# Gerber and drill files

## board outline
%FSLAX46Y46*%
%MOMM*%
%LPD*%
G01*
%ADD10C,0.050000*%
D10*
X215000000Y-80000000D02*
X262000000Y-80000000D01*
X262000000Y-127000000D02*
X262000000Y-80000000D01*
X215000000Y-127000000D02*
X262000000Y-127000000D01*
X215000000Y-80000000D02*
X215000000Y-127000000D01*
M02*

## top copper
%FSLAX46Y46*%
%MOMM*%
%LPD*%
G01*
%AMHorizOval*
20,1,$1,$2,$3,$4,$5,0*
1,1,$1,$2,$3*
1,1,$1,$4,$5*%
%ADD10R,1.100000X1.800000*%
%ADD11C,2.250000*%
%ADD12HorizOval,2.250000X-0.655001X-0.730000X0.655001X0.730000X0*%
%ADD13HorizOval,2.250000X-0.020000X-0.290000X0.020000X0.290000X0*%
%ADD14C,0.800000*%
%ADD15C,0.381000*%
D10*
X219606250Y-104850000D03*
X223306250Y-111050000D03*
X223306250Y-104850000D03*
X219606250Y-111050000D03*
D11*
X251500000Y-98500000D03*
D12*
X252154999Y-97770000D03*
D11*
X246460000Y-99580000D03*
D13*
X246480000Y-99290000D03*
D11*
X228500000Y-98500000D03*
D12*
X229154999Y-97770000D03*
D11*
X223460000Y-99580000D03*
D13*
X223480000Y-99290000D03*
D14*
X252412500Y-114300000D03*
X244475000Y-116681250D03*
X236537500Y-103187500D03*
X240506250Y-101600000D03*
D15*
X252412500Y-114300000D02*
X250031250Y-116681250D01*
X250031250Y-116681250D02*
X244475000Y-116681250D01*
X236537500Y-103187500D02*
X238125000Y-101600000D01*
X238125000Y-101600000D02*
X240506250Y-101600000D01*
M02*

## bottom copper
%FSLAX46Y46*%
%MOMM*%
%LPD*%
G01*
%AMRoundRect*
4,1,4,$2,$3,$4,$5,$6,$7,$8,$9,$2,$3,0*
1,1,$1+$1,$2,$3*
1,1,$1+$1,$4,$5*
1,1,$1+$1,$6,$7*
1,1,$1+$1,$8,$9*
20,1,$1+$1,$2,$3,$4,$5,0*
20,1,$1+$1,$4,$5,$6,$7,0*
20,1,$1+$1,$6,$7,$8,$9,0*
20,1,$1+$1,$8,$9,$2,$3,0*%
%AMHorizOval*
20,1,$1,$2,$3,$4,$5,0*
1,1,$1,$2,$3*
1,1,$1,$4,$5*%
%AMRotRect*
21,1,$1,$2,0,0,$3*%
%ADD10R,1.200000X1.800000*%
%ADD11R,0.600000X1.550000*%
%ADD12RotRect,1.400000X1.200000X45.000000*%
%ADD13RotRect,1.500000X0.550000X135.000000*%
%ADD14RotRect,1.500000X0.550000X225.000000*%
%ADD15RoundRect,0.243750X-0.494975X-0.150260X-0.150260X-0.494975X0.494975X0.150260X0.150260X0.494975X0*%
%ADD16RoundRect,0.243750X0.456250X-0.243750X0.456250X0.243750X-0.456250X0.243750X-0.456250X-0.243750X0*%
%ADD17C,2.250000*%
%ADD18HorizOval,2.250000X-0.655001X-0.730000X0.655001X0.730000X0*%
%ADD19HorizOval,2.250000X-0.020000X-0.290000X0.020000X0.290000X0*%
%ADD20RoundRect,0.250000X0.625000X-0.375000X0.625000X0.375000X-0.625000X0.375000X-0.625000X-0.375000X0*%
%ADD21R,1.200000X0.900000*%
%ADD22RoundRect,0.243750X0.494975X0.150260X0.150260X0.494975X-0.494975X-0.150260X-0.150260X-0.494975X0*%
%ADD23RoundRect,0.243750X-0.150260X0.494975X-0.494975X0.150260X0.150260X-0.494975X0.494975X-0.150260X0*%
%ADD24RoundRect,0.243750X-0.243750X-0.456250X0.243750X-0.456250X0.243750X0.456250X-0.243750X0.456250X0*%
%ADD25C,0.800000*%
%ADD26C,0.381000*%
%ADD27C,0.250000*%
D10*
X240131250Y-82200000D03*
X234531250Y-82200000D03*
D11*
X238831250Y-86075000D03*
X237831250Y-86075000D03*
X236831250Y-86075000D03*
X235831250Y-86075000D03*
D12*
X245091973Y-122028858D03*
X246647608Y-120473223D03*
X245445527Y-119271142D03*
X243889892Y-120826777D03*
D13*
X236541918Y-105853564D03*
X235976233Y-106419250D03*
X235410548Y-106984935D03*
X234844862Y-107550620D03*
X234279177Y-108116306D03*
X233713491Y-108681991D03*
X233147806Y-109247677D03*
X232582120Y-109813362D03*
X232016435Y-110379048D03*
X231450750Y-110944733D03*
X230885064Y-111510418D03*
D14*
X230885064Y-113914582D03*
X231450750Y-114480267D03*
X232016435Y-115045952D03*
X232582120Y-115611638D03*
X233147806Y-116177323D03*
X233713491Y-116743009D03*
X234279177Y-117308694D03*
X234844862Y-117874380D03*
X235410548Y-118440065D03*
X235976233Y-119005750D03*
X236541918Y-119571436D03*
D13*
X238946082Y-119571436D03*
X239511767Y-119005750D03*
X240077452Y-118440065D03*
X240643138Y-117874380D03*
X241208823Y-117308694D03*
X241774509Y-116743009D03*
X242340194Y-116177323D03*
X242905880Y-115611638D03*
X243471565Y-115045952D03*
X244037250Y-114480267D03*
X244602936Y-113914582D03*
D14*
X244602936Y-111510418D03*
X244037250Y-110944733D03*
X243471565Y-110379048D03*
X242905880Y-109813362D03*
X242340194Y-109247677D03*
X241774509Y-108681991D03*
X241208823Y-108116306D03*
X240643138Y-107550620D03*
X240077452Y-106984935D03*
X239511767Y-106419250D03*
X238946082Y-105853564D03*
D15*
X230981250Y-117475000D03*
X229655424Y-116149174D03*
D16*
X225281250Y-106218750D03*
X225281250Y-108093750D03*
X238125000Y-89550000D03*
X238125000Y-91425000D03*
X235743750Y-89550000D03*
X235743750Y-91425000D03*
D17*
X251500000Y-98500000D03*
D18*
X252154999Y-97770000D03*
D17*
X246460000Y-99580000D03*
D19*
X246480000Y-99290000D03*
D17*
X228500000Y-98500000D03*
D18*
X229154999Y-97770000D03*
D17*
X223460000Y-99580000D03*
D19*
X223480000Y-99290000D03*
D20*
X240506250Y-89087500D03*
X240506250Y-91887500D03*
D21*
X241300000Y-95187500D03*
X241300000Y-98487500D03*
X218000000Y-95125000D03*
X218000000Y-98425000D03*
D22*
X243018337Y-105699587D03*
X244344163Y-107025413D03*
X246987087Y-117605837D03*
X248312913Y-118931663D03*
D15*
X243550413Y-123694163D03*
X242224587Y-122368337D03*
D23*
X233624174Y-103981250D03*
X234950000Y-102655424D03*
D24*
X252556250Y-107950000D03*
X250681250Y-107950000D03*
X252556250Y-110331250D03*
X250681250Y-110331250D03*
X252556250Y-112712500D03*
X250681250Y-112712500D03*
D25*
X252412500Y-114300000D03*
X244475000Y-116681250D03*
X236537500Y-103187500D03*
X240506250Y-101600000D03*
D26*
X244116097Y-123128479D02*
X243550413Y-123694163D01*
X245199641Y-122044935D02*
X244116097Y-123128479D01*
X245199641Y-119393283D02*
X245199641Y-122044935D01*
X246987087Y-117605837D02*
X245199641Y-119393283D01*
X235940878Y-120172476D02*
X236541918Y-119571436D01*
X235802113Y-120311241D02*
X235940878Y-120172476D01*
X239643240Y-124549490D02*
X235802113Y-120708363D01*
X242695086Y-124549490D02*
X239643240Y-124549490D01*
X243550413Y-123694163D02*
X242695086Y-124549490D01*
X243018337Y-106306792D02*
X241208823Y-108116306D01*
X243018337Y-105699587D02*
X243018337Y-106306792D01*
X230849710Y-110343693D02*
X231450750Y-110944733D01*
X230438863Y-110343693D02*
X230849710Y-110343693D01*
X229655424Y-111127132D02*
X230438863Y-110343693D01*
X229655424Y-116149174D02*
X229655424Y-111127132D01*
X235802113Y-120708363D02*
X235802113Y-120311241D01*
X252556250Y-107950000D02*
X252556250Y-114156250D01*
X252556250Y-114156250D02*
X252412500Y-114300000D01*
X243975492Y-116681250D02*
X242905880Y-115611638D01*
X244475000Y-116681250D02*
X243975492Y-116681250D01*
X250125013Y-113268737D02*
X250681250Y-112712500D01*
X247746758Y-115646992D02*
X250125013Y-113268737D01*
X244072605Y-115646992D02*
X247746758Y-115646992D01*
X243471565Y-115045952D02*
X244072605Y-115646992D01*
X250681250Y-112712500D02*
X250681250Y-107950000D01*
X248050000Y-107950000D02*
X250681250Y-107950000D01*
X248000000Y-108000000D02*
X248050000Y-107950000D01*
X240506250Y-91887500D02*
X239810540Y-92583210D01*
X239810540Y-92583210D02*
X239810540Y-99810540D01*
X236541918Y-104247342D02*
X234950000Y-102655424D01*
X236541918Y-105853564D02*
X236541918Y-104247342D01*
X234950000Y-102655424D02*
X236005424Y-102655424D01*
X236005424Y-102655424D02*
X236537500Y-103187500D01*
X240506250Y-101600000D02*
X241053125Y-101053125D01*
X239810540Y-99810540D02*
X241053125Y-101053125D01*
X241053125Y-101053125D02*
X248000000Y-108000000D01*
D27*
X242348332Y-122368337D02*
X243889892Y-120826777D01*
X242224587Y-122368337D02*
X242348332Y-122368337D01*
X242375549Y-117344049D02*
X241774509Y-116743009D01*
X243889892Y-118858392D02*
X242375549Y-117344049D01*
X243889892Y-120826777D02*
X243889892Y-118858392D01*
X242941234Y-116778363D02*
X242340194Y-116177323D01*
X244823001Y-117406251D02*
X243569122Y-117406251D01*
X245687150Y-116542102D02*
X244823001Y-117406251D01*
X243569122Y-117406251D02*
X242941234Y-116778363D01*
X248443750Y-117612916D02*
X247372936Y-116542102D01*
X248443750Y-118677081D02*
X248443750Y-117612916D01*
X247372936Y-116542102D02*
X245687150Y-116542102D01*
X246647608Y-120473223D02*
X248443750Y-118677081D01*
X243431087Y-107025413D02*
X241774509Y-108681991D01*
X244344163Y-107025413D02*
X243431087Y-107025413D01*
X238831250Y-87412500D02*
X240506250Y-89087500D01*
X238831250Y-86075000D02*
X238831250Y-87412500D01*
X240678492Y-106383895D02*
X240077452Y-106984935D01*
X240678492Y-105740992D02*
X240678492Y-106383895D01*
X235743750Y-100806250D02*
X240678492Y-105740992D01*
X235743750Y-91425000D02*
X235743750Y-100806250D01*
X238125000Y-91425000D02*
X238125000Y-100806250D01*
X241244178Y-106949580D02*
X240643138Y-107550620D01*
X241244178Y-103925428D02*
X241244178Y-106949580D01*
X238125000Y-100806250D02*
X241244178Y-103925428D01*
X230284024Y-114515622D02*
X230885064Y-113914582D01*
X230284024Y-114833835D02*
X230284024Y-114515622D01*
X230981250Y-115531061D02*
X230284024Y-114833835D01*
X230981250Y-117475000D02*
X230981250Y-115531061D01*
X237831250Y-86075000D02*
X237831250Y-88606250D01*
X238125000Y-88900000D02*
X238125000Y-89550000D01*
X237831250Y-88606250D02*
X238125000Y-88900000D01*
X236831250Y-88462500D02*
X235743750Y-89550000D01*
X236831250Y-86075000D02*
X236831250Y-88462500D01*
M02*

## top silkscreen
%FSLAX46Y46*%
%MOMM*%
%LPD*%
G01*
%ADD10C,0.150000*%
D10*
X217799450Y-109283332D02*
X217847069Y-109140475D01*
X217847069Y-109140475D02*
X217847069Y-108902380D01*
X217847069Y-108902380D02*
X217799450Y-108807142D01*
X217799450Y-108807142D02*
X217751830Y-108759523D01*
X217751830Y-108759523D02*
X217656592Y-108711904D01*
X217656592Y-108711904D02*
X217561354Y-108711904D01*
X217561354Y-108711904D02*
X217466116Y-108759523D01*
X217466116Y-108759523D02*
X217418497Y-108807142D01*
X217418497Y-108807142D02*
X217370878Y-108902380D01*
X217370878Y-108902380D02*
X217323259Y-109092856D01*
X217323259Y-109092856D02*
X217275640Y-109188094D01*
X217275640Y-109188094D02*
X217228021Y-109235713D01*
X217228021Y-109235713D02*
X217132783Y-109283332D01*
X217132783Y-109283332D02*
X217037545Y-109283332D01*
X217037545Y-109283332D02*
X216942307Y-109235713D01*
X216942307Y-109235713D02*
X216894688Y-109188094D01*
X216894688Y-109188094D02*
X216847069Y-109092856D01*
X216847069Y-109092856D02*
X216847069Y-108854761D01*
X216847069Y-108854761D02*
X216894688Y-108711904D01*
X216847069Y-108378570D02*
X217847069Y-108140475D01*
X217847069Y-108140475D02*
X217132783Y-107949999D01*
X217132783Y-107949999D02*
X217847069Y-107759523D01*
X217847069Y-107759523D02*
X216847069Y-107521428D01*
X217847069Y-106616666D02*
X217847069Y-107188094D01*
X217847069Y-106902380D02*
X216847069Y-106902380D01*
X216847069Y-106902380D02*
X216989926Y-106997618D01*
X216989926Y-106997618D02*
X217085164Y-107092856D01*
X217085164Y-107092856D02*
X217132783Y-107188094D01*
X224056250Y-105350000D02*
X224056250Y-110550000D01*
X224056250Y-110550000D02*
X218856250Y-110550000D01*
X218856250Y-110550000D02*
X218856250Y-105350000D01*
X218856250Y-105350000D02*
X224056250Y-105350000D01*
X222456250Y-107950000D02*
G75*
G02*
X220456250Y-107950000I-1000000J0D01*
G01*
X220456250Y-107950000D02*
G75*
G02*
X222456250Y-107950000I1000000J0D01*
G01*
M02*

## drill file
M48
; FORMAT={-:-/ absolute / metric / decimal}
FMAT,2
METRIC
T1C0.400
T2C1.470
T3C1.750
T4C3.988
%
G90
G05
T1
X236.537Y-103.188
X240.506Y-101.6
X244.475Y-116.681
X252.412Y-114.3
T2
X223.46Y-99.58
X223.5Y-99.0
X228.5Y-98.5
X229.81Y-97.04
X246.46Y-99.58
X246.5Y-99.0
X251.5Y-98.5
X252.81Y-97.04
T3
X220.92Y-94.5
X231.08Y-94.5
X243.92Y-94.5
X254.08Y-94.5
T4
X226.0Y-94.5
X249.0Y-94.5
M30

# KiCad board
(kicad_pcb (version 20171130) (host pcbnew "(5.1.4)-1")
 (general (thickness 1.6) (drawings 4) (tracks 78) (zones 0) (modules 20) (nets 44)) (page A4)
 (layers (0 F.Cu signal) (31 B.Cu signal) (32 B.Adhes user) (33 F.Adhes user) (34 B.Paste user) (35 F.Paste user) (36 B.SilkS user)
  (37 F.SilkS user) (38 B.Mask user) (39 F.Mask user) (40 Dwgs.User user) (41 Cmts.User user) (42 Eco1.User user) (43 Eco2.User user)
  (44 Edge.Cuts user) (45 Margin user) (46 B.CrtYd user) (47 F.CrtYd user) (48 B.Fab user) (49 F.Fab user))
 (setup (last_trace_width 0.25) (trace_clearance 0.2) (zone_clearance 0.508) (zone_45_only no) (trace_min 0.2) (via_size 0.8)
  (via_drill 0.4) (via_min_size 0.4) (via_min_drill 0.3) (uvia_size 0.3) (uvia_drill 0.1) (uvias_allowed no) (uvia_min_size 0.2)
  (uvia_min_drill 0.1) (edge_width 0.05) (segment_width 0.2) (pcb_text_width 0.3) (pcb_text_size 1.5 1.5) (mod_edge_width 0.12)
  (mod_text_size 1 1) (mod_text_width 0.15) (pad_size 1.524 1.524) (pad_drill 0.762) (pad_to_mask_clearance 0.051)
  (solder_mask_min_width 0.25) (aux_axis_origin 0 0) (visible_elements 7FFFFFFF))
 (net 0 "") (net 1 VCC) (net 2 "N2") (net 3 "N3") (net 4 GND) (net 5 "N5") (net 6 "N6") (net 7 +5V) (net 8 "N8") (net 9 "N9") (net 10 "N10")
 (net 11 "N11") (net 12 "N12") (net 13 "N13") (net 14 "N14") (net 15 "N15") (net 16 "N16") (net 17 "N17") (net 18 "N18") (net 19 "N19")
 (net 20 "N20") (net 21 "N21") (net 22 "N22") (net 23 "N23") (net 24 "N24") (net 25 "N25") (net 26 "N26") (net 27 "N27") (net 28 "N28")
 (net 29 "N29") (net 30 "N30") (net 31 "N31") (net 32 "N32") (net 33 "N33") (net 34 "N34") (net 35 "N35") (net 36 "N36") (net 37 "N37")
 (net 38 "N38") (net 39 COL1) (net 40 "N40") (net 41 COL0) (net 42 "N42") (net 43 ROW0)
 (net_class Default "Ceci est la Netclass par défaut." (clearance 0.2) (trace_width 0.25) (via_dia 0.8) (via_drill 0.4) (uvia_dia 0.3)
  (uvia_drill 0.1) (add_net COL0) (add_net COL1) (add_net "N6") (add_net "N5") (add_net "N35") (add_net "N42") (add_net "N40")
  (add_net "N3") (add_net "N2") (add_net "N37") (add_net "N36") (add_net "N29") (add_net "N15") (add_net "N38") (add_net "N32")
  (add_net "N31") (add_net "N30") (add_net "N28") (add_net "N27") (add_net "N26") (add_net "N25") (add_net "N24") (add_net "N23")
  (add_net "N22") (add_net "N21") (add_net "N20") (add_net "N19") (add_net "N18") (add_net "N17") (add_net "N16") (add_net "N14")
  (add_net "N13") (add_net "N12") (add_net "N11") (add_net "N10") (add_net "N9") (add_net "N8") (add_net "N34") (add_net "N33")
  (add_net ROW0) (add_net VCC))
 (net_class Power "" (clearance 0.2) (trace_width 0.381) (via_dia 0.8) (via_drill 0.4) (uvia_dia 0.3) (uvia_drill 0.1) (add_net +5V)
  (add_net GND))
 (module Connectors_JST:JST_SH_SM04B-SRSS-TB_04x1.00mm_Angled (layer B.Cu) (at 237.33125 84.1375)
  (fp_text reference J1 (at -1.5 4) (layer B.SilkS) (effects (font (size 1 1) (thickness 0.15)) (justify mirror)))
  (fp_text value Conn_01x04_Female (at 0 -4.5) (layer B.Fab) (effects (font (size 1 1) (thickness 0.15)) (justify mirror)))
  (pad "" smd rect (at 2.8 -1.9375) (size 1.2 1.8) (layers B.Cu B.Paste B.Mask))
  (pad "" smd rect (at -2.8 -1.9375) (size 1.2 1.8) (layers B.Cu B.Paste B.Mask))
  (pad 4 smd rect (at 1.5 1.9375) (size 0.6 1.55) (layers B.Cu B.Paste B.Mask) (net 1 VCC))
  (pad 3 smd rect (at 0.5 1.9375) (size 0.6 1.55) (layers B.Cu B.Paste B.Mask) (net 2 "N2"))
  (pad 2 smd rect (at -0.5 1.9375) (size 0.6 1.55) (layers B.Cu B.Paste B.Mask) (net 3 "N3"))
  (pad 1 smd rect (at -1.5 1.9375) (size 0.6 1.55) (layers B.Cu B.Paste B.Mask) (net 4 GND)))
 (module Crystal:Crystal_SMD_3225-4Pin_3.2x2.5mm (layer B.Cu) (at 245.26875 120.65 45)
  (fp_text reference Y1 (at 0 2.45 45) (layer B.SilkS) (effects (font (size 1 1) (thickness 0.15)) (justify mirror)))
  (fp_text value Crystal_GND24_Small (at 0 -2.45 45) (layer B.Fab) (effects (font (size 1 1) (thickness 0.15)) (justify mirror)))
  (pad 4 smd rect (at -1.1 0.85 45) (size 1.4 1.2) (layers B.Cu B.Paste B.Mask) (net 4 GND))
  (pad 3 smd rect (at 1.1 0.85 45) (size 1.4 1.2) (layers B.Cu B.Paste B.Mask) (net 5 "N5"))
  (pad 2 smd rect (at 1.1 -0.85 45) (size 1.4 1.2) (layers B.Cu B.Paste B.Mask) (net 4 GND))
  (pad 1 smd rect (at -1.1 -0.85 45) (size 1.4 1.2) (layers B.Cu B.Paste B.Mask) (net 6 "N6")))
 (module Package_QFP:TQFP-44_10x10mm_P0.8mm (layer B.Cu) (at 237.744 112.7125 225)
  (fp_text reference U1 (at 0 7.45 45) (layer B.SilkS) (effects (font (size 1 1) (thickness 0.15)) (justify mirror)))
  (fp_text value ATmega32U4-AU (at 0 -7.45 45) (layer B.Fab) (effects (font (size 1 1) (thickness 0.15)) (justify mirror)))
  (pad 44 smd rect (at -4 5.7 135) (size 1.5 0.55) (layers B.Cu B.Paste B.Mask) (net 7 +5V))
  (pad 43 smd rect (at -3.2 5.7 135) (size 1.5 0.55) (layers B.Cu B.Paste B.Mask) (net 4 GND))
  (pad 42 smd rect (at -2.4 5.7 135) (size 1.5 0.55) (layers B.Cu B.Paste B.Mask) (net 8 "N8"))
  (pad 41 smd rect (at -1.6 5.7 135) (size 1.5 0.55) (layers B.Cu B.Paste B.Mask) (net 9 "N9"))
  (pad 40 smd rect (at -0.8 5.7 135) (size 1.5 0.55) (layers B.Cu B.Paste B.Mask) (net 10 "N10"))
  (pad 39 smd rect (at 0 5.7 135) (size 1.5 0.55) (layers B.Cu B.Paste B.Mask) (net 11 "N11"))
  (pad 38 smd rect (at 0.8 5.7 135) (size 1.5 0.55) (layers B.Cu B.Paste B.Mask) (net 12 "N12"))
  (pad 37 smd rect (at 1.6 5.7 135) (size 1.5 0.55) (layers B.Cu B.Paste B.Mask) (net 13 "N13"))
  (pad 36 smd rect (at 2.4 5.7 135) (size 1.5 0.55) (layers B.Cu B.Paste B.Mask) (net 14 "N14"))
  (pad 35 smd rect (at 3.2 5.7 135) (size 1.5 0.55) (layers B.Cu B.Paste B.Mask) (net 4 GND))
  (pad 34 smd rect (at 4 5.7 135) (size 1.5 0.55) (layers B.Cu B.Paste B.Mask) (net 7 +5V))
  (pad 33 smd rect (at 5.7 4 225) (size 1.5 0.55) (layers B.Cu B.Paste B.Mask) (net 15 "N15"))
  (pad 32 smd rect (at 5.7 3.2 225) (size 1.5 0.55) (layers B.Cu B.Paste B.Mask) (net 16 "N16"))
  (pad 31 smd rect (at 5.7 2.4 225) (size 1.5 0.55) (layers B.Cu B.Paste B.Mask) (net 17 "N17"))
  (pad 30 smd rect (at 5.7 1.6 225) (size 1.5 0.55) (layers B.Cu B.Paste B.Mask) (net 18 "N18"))
  (pad 29 smd rect (at 5.7 0.8 225) (size 1.5 0.55) (layers B.Cu B.Paste B.Mask) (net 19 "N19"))
  (pad 28 smd rect (at 5.7 0 225) (size 1.5 0.55) (layers B.Cu B.Paste B.Mask) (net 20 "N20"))
  (pad 27 smd rect (at 5.7 -0.8 225) (size 1.5 0.55) (layers B.Cu B.Paste B.Mask) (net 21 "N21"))
  (pad 26 smd rect (at 5.7 -1.6 225) (size 1.5 0.55) (layers B.Cu B.Paste B.Mask) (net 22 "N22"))
  (pad 25 smd rect (at 5.7 -2.4 225) (size 1.5 0.55) (layers B.Cu B.Paste B.Mask) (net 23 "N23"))
  (pad 24 smd rect (at 5.7 -3.2 225) (size 1.5 0.55) (layers B.Cu B.Paste B.Mask) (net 7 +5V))
  (pad 23 smd rect (at 5.7 -4 225) (size 1.5 0.55) (layers B.Cu B.Paste B.Mask) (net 4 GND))
  (pad 22 smd rect (at 4 -5.7 135) (size 1.5 0.55) (layers B.Cu B.Paste B.Mask) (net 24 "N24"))
  (pad 21 smd rect (at 3.2 -5.7 135) (size 1.5 0.55) (layers B.Cu B.Paste B.Mask) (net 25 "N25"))
  (pad 20 smd rect (at 2.4 -5.7 135) (size 1.5 0.55) (layers B.Cu B.Paste B.Mask) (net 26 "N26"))
  (pad 19 smd rect (at 1.6 -5.7 135) (size 1.5 0.55) (layers B.Cu B.Paste B.Mask) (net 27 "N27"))
  (pad 18 smd rect (at 0.8 -5.7 135) (size 1.5 0.55) (layers B.Cu B.Paste B.Mask) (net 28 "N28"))
  (pad 17 smd rect (at 0 -5.7 135) (size 1.5 0.55) (layers B.Cu B.Paste B.Mask) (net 6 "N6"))
  (pad 16 smd rect (at -0.8 -5.7 135) (size 1.5 0.55) (layers B.Cu B.Paste B.Mask) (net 5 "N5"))
  (pad 15 smd rect (at -1.6 -5.7 135) (size 1.5 0.55) (layers B.Cu B.Paste B.Mask) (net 4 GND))
  (pad 14 smd rect (at -2.4 -5.7 135) (size 1.5 0.55) (layers B.Cu B.Paste B.Mask) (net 7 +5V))
  (pad 13 smd rect (at -3.2 -5.7 135) (size 1.5 0.55) (layers B.Cu B.Paste B.Mask) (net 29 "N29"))
  (pad 12 smd rect (at -4 -5.7 135) (size 1.5 0.55) (layers B.Cu B.Paste B.Mask) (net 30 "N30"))
  (pad 11 smd rect (at -5.7 -4 225) (size 1.5 0.55) (layers B.Cu B.Paste B.Mask) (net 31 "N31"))
  (pad 10 smd rect (at -5.7 -3.2 225) (size 1.5 0.55) (layers B.Cu B.Paste B.Mask) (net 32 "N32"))
  (pad 9 smd rect (at -5.7 -2.4 225) (size 1.5 0.55) (layers B.Cu B.Paste B.Mask) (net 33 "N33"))
  (pad 8 smd rect (at -5.7 -1.6 225) (size 1.5 0.55) (layers B.Cu B.Paste B.Mask) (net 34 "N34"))
  (pad 7 smd rect (at -5.7 -0.8 225) (size 1.5 0.55) (layers B.Cu B.Paste B.Mask) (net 7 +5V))
  (pad 6 smd rect (at -5.7 0 225) (size 1.5 0.55) (layers B.Cu B.Paste B.Mask) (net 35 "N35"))
  (pad 5 smd rect (at -5.7 0.8 225) (size 1.5 0.55) (layers B.Cu B.Paste B.Mask) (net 4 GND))
  (pad 4 smd rect (at -5.7 1.6 225) (size 1.5 0.55) (layers B.Cu B.Paste B.Mask) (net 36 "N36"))
  (pad 3 smd rect (at -5.7 2.4 225) (size 1.5 0.55) (layers B.Cu B.Paste B.Mask) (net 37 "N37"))
  (pad 2 smd rect (at -5.7 3.2 225) (size 1.5 0.55) (layers B.Cu B.Paste B.Mask) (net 7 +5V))
  (pad 1 smd rect (at -5.7 4 225) (size 1.5 0.55) (layers B.Cu B.Paste B.Mask) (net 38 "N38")))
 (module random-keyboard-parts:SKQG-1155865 (layer F.Cu) (at 221.45625 107.95 270)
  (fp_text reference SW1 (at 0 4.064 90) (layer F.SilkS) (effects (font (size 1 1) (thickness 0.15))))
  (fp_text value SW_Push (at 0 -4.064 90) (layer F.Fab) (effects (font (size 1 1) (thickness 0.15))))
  (fp_line (start -2.6 -2.6) (end 2.6 -2.6) (layer F.SilkS) (width 0.15))
  (fp_line (start 2.6 -2.6) (end 2.6 2.6) (layer F.SilkS) (width 0.15))
  (fp_line (start 2.6 2.6) (end -2.6 2.6) (layer F.SilkS) (width 0.15))
  (fp_line (start -2.6 2.6) (end -2.6 -2.6) (layer F.SilkS) (width 0.15))
  (fp_circle (center 0 0) (end 1 0) (layer F.SilkS) (width 0.15))
  (pad 4 smd rect (at -3.1 1.85 270) (size 1.8 1.1) (layers F.Cu F.Paste F.Mask))
  (pad 3 smd rect (at 3.1 -1.85 270) (size 1.8 1.1) (layers F.Cu F.Paste F.Mask))
  (pad 2 smd rect (at -3.1 -1.85 270) (size 1.8 1.1) (layers F.Cu F.Paste F.Mask) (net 29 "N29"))
  (pad 1 smd rect (at 3.1 1.85 270) (size 1.8 1.1) (layers F.Cu F.Paste F.Mask) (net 4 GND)))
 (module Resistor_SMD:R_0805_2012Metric (layer B.Cu) (at 230.318337 116.812087 315)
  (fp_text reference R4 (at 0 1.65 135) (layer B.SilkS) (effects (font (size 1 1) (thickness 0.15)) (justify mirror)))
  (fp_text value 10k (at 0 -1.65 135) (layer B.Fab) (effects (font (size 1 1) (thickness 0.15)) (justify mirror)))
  (pad 2 smd roundrect (at 0.9375 0 315) (size 0.975 1.4) (layers B.Cu B.Paste B.Mask) (roundrect_rratio 0.25) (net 15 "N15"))
  (pad 1 smd roundrect (at -0.9375 0 315) (size 0.975 1.4) (layers B.Cu B.Paste B.Mask) (roundrect_rratio 0.25) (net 4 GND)))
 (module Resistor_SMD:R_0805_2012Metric (layer B.Cu) (at 225.28125 107.15625 90)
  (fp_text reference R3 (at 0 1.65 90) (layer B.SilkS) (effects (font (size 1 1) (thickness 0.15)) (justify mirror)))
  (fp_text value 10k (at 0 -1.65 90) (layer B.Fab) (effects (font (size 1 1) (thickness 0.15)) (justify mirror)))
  (pad 2 smd roundrect (at 0.9375 0 90) (size 0.975 1.4) (layers B.Cu B.Paste B.Mask) (roundrect_rratio 0.25) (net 29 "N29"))
  (pad 1 smd roundrect (at -0.9375 0 90) (size 0.975 1.4) (layers B.Cu B.Paste B.Mask) (roundrect_rratio 0.25) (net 7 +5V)))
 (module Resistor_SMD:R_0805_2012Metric (layer B.Cu) (at 238.125 90.4875 90)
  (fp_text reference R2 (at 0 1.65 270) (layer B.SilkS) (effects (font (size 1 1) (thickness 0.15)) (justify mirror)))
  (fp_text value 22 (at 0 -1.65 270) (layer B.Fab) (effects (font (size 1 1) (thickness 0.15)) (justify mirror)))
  (pad 2 smd roundrect (at 0.9375 0 90) (size 0.975 1.4) (layers B.Cu B.Paste B.Mask) (roundrect_rratio 0.25) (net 2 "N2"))
  (pad 1 smd roundrect (at -0.9375 0 90) (size 0.975 1.4) (layers B.Cu B.Paste B.Mask) (roundrect_rratio 0.25) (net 36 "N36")))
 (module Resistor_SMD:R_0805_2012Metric (layer B.Cu) (at 235.74375 90.4875 90)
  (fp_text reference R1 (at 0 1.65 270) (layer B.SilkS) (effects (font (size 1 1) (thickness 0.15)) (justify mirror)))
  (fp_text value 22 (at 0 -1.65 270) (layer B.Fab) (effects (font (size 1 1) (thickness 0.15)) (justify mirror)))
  (pad 2 smd roundrect (at 0.9375 0 90) (size 0.975 1.4) (layers B.Cu B.Paste B.Mask) (roundrect_rratio 0.25) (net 3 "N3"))
  (pad 1 smd roundrect (at -0.9375 0 90) (size 0.975 1.4) (layers B.Cu B.Paste B.Mask) (roundrect_rratio 0.25) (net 37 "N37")))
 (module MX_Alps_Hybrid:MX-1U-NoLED (layer F.Cu) (at 249 94.5 180)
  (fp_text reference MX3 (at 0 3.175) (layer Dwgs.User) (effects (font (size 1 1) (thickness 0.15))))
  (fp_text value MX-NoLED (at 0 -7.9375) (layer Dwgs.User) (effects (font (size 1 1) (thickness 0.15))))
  (pad "" np_thru_hole circle (at 5.08 0 228.0996) (size 1.75 1.75) (drill 1.75) (layers *.Cu *.Mask))
  (pad "" np_thru_hole circle (at -5.08 0 228.0996) (size 1.75 1.75) (drill 1.75) (layers *.Cu *.Mask))
  (pad 1 thru_hole circle (at -2.5 -4 180) (size 2.25 2.25) (drill 1.47) (layers *.Cu B.Mask) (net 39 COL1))
  (pad "" np_thru_hole circle (at 0 0 180) (size 3.9878 3.9878) (drill 3.9878) (layers *.Cu *.Mask))
  (pad 1 thru_hole oval (at -3.81 -2.54 228.0996) (size 4.211556 2.25) (drill 1.47 (offset 0.980778 0)) (layers *.Cu B.Mask) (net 39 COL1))
  (pad 2 thru_hole circle (at 2.54 -5.08 180) (size 2.25 2.25) (drill 1.47) (layers *.Cu B.Mask) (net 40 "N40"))
  (pad 2 thru_hole oval (at 2.5 -4.5 266.0548) (size 2.831378 2.25) (drill 1.47 (offset 0.290689 0)) (layers *.Cu B.Mask) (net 40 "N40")))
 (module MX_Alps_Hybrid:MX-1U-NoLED (layer F.Cu) (at 226 94.5 180)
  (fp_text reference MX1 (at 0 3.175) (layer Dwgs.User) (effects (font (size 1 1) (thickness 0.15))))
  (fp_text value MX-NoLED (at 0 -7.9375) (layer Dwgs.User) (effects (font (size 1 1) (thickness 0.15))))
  (pad "" np_thru_hole circle (at 5.08 0 228.0996) (size 1.75 1.75) (drill 1.75) (layers *.Cu *.Mask))
  (pad "" np_thru_hole circle (at -5.08 0 228.0996) (size 1.75 1.75) (drill 1.75) (layers *.Cu *.Mask))
  (pad 1 thru_hole circle (at -2.5 -4 180) (size 2.25 2.25) (drill 1.47) (layers *.Cu B.Mask) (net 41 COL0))
  (pad "" np_thru_hole circle (at 0 0 180) (size 3.9878 3.9878) (drill 3.9878) (layers *.Cu *.Mask))
  (pad 1 thru_hole oval (at -3.81 -2.54 228.0996) (size 4.211556 2.25) (drill 1.47 (offset 0.980778 0)) (layers *.Cu B.Mask) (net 41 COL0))
  (pad 2 thru_hole circle (at 2.54 -5.08 180) (size 2.25 2.25) (drill 1.47) (layers *.Cu B.Mask) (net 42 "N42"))
  (pad 2 thru_hole oval (at 2.5 -4.5 266.0548) (size 2.831378 2.25) (drill 1.47 (offset 0.290689 0)) (layers *.Cu B.Mask) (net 42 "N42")))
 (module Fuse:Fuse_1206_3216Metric (layer B.Cu) (at 240.50625 90.4875 90)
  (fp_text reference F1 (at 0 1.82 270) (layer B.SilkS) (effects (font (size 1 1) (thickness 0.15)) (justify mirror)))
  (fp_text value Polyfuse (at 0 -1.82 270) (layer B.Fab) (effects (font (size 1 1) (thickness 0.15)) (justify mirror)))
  (pad 2 smd roundrect (at 1.4 0 90) (size 1.25 1.75) (layers B.Cu B.Paste B.Mask) (roundrect_rratio 0.2) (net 1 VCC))
  (pad 1 smd roundrect (at -1.4 0 90) (size 1.25 1.75) (layers B.Cu B.Paste B.Mask) (roundrect_rratio 0.2) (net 7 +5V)))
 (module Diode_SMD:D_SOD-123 (layer B.Cu) (at 241.3 96.8375 90)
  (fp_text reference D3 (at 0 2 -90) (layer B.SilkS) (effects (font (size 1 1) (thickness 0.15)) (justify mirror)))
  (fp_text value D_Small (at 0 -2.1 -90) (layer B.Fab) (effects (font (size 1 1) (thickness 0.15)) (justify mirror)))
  (pad 2 smd rect (at 1.65 0 90) (size 0.9 1.2) (layers B.Cu B.Paste B.Mask) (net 40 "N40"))
  (pad 1 smd rect (at -1.65 0 90) (size 0.9 1.2) (layers B.Cu B.Paste B.Mask) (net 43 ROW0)))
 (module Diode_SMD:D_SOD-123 (layer B.Cu) (at 218 96.775 90)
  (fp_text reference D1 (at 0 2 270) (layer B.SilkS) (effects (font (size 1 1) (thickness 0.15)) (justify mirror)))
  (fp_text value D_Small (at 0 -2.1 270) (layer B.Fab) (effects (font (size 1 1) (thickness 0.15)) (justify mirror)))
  (pad 2 smd rect (at 1.65 0 90) (size 0.9 1.2) (layers B.Cu B.Paste B.Mask) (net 42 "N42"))
  (pad 1 smd rect (at -1.65 0 90) (size 0.9 1.2) (layers B.Cu B.Paste B.Mask) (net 43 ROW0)))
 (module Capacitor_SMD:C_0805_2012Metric (layer B.Cu) (at 243.68125 106.3625 135)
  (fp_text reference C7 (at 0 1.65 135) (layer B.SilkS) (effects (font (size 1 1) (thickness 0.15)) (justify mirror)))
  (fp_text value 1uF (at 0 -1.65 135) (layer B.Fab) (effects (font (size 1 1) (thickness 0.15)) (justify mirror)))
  (pad 2 smd roundrect (at 0.9375 0 135) (size 0.975 1.4) (layers B.Cu B.Paste B.Mask) (roundrect_rratio 0.25) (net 4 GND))
  (pad 1 smd roundrect (at -0.9375 0 135) (size 0.975 1.4) (layers B.Cu B.Paste B.Mask) (roundrect_rratio 0.25) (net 35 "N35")))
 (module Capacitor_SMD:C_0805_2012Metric (layer B.Cu) (at 247.65 118.26875 135)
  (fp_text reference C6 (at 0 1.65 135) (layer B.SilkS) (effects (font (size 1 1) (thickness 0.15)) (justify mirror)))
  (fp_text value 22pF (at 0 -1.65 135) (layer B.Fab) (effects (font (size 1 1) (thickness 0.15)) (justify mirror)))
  (pad 2 smd roundrect (at 0.9375 0 135) (size 0.975 1.4) (layers B.Cu B.Paste B.Mask) (roundrect_rratio 0.25) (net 4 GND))
  (pad 1 smd roundrect (at -0.9375 0 135) (size 0.975 1.4) (layers B.Cu B.Paste B.Mask) (roundrect_rratio 0.25) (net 5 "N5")))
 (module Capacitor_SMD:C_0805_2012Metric (layer B.Cu) (at 242.8875 123.03125 315)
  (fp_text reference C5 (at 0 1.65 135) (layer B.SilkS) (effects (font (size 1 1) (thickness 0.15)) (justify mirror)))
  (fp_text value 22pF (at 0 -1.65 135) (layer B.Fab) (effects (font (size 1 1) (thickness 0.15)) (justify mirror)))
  (pad 2 smd roundrect (at 0.9375 0 315) (size 0.975 1.4) (layers B.Cu B.Paste B.Mask) (roundrect_rratio 0.25) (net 4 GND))
  (pad 1 smd roundrect (at -0.9375 0 315) (size 0.975 1.4) (layers B.Cu B.Paste B.Mask) (roundrect_rratio 0.25) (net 6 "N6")))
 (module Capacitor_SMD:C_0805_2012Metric (layer B.Cu) (at 234.287087 103.318337 225)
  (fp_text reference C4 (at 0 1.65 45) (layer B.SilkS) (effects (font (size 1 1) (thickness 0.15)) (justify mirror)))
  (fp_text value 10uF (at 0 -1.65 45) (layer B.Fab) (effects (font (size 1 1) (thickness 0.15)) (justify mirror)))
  (pad 2 smd roundrect (at 0.9375 0 225) (size 0.975 1.4) (layers B.Cu B.Paste B.Mask) (roundrect_rratio 0.25) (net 4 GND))
  (pad 1 smd roundrect (at -0.9375 0 225) (size 0.975 1.4) (layers B.Cu B.Paste B.Mask) (roundrect_rratio 0.25) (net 7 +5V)))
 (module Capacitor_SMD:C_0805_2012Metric (layer B.Cu) (at 251.61875 107.95)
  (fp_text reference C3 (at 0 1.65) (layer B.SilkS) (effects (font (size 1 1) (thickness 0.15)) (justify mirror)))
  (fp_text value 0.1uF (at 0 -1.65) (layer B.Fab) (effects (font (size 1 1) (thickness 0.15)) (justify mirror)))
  (pad 2 smd roundrect (at 0.9375 0) (size 0.975 1.4) (layers B.Cu B.Paste B.Mask) (roundrect_rratio 0.25) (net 4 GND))
  (pad 1 smd roundrect (at -0.9375 0) (size 0.975 1.4) (layers B.Cu B.Paste B.Mask) (roundrect_rratio 0.25) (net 7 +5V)))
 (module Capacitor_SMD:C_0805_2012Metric (layer B.Cu) (at 251.61875 110.33125)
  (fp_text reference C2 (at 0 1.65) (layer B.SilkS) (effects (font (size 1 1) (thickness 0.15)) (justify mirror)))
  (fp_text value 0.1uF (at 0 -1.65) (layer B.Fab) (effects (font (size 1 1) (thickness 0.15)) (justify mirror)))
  (pad 2 smd roundrect (at 0.9375 0) (size 0.975 1.4) (layers B.Cu B.Paste B.Mask) (roundrect_rratio 0.25) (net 4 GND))
  (pad 1 smd roundrect (at -0.9375 0) (size 0.975 1.4) (layers B.Cu B.Paste B.Mask) (roundrect_rratio 0.25) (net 7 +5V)))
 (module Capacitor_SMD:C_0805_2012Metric (layer B.Cu) (at 251.61875 112.7125)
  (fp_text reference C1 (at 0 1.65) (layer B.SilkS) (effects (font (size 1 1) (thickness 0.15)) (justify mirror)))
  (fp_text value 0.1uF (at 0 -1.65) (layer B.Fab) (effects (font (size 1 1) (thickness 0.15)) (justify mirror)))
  (pad 2 smd roundrect (at 0.9375 0) (size 0.975 1.4) (layers B.Cu B.Paste B.Mask) (roundrect_rratio 0.25) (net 4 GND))
  (pad 1 smd roundrect (at -0.9375 0) (size 0.975 1.4) (layers B.Cu B.Paste B.Mask) (roundrect_rratio 0.25) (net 7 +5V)))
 (gr_line (start 215 80) (end 262 80) (layer Edge.Cuts) (width 0.05))
 (gr_line (start 262 127) (end 262 80) (layer Edge.Cuts) (width 0.05))
 (gr_line (start 215 127) (end 262 127) (layer Edge.Cuts) (width 0.05))
 (gr_line (start 215 80) (end 215 127) (layer Edge.Cuts) (width 0.05))
 (segment (start 244.116097 123.128479) (end 243.550413 123.694163) (width 0.381) (layer B.Cu) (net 4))
 (segment (start 245.199641 122.044935) (end 244.116097 123.128479) (width 0.381) (layer B.Cu) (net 4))
 (segment (start 245.199641 119.393283) (end 245.199641 122.044935) (width 0.381) (layer B.Cu) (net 4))
 (segment (start 246.987087 117.605837) (end 245.199641 119.393283) (width 0.381) (layer B.Cu) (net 4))
 (segment (start 235.940878 120.172476) (end 236.541918 119.571436) (width 0.381) (layer B.Cu) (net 4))
 (segment (start 235.802113 120.311241) (end 235.940878 120.172476) (width 0.381) (layer B.Cu) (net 4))
 (segment (start 239.64324 124.54949) (end 235.802113 120.708363) (width 0.381) (layer B.Cu) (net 4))
 (segment (start 242.695086 124.54949) (end 239.64324 124.54949) (width 0.381) (layer B.Cu) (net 4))
 (segment (start 243.550413 123.694163) (end 242.695086 124.54949) (width 0.381) (layer B.Cu) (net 4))
 (segment (start 243.018337 106.306792) (end 241.208823 108.116306) (width 0.381) (layer B.Cu) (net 4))
 (segment (start 243.018337 105.699587) (end 243.018337 106.306792) (width 0.381) (layer B.Cu) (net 4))
 (segment (start 230.84971 110.343693) (end 231.45075 110.944733) (width 0.381) (layer B.Cu) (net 4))
 (segment (start 230.438863 110.343693) (end 230.84971 110.343693) (width 0.381) (layer B.Cu) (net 4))
 (segment (start 229.655424 111.127132) (end 230.438863 110.343693) (width 0.381) (layer B.Cu) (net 4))
 (segment (start 229.655424 116.149174) (end 229.655424 111.127132) (width 0.381) (layer B.Cu) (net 4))
 (segment (start 235.802113 120.708363) (end 235.802113 120.311241) (width 0.381) (layer B.Cu) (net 4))
 (via (at 252.4125 114.3) (size 0.8) (drill 0.4) (layers F.Cu B.Cu) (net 4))
 (segment (start 252.55625 107.95) (end 252.55625 114.15625) (width 0.381) (layer B.Cu) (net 4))
 (segment (start 252.55625 114.15625) (end 252.4125 114.3) (width 0.381) (layer B.Cu) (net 4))
 (via (at 244.475 116.68125) (size 0.8) (drill 0.4) (layers F.Cu B.Cu) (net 4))
 (segment (start 252.4125 114.3) (end 250.03125 116.68125) (width 0.381) (layer F.Cu) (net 4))
 (segment (start 250.03125 116.68125) (end 244.475 116.68125) (width 0.381) (layer F.Cu) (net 4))
 (segment (start 243.975492 116.68125) (end 242.90588 115.611638) (width 0.381) (layer B.Cu) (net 4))
 (segment (start 244.475 116.68125) (end 243.975492 116.68125) (width 0.381) (layer B.Cu) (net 4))
 (segment (start 250.125013 113.268737) (end 250.68125 112.7125) (width 0.381) (layer B.Cu) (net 7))
 (segment (start 247.746758 115.646992) (end 250.125013 113.268737) (width 0.381) (layer B.Cu) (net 7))
 (segment (start 244.072605 115.646992) (end 247.746758 115.646992) (width 0.381) (layer B.Cu) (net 7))
 (segment (start 243.471565 115.045952) (end 244.072605 115.646992) (width 0.381) (layer B.Cu) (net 7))
 (segment (start 250.68125 112.7125) (end 250.68125 107.95) (width 0.381) (layer B.Cu) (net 7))
 (segment (start 248.05 107.95) (end 250.68125 107.95) (width 0.381) (layer B.Cu) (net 7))
 (segment (start 248 108) (end 248.05 107.95) (width 0.381) (layer B.Cu) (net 7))
 (segment (start 240.50625 91.8875) (end 239.81054 92.58321) (width 0.381) (layer B.Cu) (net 7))
 (segment (start 239.81054 92.58321) (end 239.81054 99.81054) (width 0.381) (layer B.Cu) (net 7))
 (segment (start 236.541918 104.247342) (end 234.95 102.655424) (width 0.381) (layer B.Cu) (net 7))
 (segment (start 236.541918 105.853564) (end 236.541918 104.247342) (width 0.381) (layer B.Cu) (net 7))
 (via (at 236.5375 103.1875) (size 0.8) (drill 0.4) (layers F.Cu B.Cu) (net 7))
 (segment (start 234.95 102.655424) (end 236.005424 102.655424) (width 0.381) (layer B.Cu) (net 7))
 (segment (start 236.005424 102.655424) (end 236.5375 103.1875) (width 0.381) (layer B.Cu) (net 7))
 (via (at 240.50625 101.6) (size 0.8) (drill 0.4) (layers F.Cu B.Cu) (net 7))
 (segment (start 236.5375 103.1875) (end 238.125 101.6) (width 0.381) (layer F.Cu) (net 7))
 (segment (start 238.125 101.6) (end 240.50625 101.6) (width 0.381) (layer F.Cu) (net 7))
 (segment (start 240.50625 101.6) (end 241.053125 101.053125) (width 0.381) (layer B.Cu) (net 7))
 (segment (start 239.81054 99.81054) (end 241.053125 101.053125) (width 0.381) (layer B.Cu) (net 7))
 (segment (start 241.053125 101.053125) (end 248 108) (width 0.381) (layer B.Cu) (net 7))
 (segment (start 242.348332 122.368337) (end 243.889892 120.826777) (width 0.25) (layer B.Cu) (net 6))
 (segment (start 242.224587 122.368337) (end 242.348332 122.368337) (width 0.25) (layer B.Cu) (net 6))
 (segment (start 242.375549 117.344049) (end 241.774509 116.743009) (width 0.25) (layer B.Cu) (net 6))
 (segment (start 243.889892 118.858392) (end 242.375549 117.344049) (width 0.25) (layer B.Cu) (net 6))
 (segment (start 243.889892 120.826777) (end 243.889892 118.858392) (width 0.25) (layer B.Cu) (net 6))
 (segment (start 242.941234 116.778363) (end 242.340194 116.177323) (width 0.25) (layer B.Cu) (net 5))
 (segment (start 244.823001 117.406251) (end 243.569122 117.406251) (width 0.25) (layer B.Cu) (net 5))
 (segment (start 245.68715 116.542102) (end 244.823001 117.406251) (width 0.25) (layer B.Cu) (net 5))
 (segment (start 243.569122 117.406251) (end 242.941234 116.778363) (width 0.25) (layer B.Cu) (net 5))
 (segment (start 248.44375 117.612916) (end 247.372936 116.542102) (width 0.25) (layer B.Cu) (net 5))
 (segment (start 248.44375 118.677081) (end 248.44375 117.612916) (width 0.25) (layer B.Cu) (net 5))
 (segment (start 247.372936 116.542102) (end 245.68715 116.542102) (width 0.25) (layer B.Cu) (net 5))
 (segment (start 246.647608 120.473223) (end 248.44375 118.677081) (width 0.25) (layer B.Cu) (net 5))
 (segment (start 243.431087 107.025413) (end 241.774509 108.681991) (width 0.25) (layer B.Cu) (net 35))
 (segment (start 244.344163 107.025413) (end 243.431087 107.025413) (width 0.25) (layer B.Cu) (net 35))
 (segment (start 238.83125 87.4125) (end 240.50625 89.0875) (width 0.25) (layer B.Cu) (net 1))
 (segment (start 238.83125 86.075) (end 238.83125 87.4125) (width 0.25) (layer B.Cu) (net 1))
 (segment (start 240.678492 106.383895) (end 240.077452 106.984935) (width 0.25) (layer B.Cu) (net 37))
 (segment (start 240.678492 105.740992) (end 240.678492 106.383895) (width 0.25) (layer B.Cu) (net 37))
 (segment (start 235.74375 100.80625) (end 240.678492 105.740992) (width 0.25) (layer B.Cu) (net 37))
 (segment (start 235.74375 91.425) (end 235.74375 100.80625) (width 0.25) (layer B.Cu) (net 37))
 (segment (start 238.125 91.425) (end 238.125 100.80625) (width 0.25) (layer B.Cu) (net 36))
 (segment (start 241.244178 106.94958) (end 240.643138 107.55062) (width 0.25) (layer B.Cu) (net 36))
 (segment (start 241.244178 103.925428) (end 241.244178 106.94958) (width 0.25) (layer B.Cu) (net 36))
 (segment (start 238.125 100.80625) (end 241.244178 103.925428) (width 0.25) (layer B.Cu) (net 36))
 (segment (start 230.284024 114.515622) (end 230.885064 113.914582) (width 0.25) (layer B.Cu) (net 15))
 (segment (start 230.284024 114.833835) (end 230.284024 114.515622) (width 0.25) (layer B.Cu) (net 15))
 (segment (start 230.98125 115.531061) (end 230.284024 114.833835) (width 0.25) (layer B.Cu) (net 15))
 (segment (start 230.98125 117.475) (end 230.98125 115.531061) (width 0.25) (layer B.Cu) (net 15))
 (segment (start 237.83125 86.075) (end 237.83125 88.60625) (width 0.25) (layer B.Cu) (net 2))
 (segment (start 238.125 88.9) (end 238.125 89.55) (width 0.25) (layer B.Cu) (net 2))
 (segment (start 237.83125 88.60625) (end 238.125 88.9) (width 0.25) (layer B.Cu) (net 2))
 (segment (start 236.83125 88.4625) (end 235.74375 89.55) (width 0.25) (layer B.Cu) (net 3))
 (segment (start 236.83125 86.075) (end 236.83125 88.4625) (width 0.25) (layer B.Cu) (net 3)))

